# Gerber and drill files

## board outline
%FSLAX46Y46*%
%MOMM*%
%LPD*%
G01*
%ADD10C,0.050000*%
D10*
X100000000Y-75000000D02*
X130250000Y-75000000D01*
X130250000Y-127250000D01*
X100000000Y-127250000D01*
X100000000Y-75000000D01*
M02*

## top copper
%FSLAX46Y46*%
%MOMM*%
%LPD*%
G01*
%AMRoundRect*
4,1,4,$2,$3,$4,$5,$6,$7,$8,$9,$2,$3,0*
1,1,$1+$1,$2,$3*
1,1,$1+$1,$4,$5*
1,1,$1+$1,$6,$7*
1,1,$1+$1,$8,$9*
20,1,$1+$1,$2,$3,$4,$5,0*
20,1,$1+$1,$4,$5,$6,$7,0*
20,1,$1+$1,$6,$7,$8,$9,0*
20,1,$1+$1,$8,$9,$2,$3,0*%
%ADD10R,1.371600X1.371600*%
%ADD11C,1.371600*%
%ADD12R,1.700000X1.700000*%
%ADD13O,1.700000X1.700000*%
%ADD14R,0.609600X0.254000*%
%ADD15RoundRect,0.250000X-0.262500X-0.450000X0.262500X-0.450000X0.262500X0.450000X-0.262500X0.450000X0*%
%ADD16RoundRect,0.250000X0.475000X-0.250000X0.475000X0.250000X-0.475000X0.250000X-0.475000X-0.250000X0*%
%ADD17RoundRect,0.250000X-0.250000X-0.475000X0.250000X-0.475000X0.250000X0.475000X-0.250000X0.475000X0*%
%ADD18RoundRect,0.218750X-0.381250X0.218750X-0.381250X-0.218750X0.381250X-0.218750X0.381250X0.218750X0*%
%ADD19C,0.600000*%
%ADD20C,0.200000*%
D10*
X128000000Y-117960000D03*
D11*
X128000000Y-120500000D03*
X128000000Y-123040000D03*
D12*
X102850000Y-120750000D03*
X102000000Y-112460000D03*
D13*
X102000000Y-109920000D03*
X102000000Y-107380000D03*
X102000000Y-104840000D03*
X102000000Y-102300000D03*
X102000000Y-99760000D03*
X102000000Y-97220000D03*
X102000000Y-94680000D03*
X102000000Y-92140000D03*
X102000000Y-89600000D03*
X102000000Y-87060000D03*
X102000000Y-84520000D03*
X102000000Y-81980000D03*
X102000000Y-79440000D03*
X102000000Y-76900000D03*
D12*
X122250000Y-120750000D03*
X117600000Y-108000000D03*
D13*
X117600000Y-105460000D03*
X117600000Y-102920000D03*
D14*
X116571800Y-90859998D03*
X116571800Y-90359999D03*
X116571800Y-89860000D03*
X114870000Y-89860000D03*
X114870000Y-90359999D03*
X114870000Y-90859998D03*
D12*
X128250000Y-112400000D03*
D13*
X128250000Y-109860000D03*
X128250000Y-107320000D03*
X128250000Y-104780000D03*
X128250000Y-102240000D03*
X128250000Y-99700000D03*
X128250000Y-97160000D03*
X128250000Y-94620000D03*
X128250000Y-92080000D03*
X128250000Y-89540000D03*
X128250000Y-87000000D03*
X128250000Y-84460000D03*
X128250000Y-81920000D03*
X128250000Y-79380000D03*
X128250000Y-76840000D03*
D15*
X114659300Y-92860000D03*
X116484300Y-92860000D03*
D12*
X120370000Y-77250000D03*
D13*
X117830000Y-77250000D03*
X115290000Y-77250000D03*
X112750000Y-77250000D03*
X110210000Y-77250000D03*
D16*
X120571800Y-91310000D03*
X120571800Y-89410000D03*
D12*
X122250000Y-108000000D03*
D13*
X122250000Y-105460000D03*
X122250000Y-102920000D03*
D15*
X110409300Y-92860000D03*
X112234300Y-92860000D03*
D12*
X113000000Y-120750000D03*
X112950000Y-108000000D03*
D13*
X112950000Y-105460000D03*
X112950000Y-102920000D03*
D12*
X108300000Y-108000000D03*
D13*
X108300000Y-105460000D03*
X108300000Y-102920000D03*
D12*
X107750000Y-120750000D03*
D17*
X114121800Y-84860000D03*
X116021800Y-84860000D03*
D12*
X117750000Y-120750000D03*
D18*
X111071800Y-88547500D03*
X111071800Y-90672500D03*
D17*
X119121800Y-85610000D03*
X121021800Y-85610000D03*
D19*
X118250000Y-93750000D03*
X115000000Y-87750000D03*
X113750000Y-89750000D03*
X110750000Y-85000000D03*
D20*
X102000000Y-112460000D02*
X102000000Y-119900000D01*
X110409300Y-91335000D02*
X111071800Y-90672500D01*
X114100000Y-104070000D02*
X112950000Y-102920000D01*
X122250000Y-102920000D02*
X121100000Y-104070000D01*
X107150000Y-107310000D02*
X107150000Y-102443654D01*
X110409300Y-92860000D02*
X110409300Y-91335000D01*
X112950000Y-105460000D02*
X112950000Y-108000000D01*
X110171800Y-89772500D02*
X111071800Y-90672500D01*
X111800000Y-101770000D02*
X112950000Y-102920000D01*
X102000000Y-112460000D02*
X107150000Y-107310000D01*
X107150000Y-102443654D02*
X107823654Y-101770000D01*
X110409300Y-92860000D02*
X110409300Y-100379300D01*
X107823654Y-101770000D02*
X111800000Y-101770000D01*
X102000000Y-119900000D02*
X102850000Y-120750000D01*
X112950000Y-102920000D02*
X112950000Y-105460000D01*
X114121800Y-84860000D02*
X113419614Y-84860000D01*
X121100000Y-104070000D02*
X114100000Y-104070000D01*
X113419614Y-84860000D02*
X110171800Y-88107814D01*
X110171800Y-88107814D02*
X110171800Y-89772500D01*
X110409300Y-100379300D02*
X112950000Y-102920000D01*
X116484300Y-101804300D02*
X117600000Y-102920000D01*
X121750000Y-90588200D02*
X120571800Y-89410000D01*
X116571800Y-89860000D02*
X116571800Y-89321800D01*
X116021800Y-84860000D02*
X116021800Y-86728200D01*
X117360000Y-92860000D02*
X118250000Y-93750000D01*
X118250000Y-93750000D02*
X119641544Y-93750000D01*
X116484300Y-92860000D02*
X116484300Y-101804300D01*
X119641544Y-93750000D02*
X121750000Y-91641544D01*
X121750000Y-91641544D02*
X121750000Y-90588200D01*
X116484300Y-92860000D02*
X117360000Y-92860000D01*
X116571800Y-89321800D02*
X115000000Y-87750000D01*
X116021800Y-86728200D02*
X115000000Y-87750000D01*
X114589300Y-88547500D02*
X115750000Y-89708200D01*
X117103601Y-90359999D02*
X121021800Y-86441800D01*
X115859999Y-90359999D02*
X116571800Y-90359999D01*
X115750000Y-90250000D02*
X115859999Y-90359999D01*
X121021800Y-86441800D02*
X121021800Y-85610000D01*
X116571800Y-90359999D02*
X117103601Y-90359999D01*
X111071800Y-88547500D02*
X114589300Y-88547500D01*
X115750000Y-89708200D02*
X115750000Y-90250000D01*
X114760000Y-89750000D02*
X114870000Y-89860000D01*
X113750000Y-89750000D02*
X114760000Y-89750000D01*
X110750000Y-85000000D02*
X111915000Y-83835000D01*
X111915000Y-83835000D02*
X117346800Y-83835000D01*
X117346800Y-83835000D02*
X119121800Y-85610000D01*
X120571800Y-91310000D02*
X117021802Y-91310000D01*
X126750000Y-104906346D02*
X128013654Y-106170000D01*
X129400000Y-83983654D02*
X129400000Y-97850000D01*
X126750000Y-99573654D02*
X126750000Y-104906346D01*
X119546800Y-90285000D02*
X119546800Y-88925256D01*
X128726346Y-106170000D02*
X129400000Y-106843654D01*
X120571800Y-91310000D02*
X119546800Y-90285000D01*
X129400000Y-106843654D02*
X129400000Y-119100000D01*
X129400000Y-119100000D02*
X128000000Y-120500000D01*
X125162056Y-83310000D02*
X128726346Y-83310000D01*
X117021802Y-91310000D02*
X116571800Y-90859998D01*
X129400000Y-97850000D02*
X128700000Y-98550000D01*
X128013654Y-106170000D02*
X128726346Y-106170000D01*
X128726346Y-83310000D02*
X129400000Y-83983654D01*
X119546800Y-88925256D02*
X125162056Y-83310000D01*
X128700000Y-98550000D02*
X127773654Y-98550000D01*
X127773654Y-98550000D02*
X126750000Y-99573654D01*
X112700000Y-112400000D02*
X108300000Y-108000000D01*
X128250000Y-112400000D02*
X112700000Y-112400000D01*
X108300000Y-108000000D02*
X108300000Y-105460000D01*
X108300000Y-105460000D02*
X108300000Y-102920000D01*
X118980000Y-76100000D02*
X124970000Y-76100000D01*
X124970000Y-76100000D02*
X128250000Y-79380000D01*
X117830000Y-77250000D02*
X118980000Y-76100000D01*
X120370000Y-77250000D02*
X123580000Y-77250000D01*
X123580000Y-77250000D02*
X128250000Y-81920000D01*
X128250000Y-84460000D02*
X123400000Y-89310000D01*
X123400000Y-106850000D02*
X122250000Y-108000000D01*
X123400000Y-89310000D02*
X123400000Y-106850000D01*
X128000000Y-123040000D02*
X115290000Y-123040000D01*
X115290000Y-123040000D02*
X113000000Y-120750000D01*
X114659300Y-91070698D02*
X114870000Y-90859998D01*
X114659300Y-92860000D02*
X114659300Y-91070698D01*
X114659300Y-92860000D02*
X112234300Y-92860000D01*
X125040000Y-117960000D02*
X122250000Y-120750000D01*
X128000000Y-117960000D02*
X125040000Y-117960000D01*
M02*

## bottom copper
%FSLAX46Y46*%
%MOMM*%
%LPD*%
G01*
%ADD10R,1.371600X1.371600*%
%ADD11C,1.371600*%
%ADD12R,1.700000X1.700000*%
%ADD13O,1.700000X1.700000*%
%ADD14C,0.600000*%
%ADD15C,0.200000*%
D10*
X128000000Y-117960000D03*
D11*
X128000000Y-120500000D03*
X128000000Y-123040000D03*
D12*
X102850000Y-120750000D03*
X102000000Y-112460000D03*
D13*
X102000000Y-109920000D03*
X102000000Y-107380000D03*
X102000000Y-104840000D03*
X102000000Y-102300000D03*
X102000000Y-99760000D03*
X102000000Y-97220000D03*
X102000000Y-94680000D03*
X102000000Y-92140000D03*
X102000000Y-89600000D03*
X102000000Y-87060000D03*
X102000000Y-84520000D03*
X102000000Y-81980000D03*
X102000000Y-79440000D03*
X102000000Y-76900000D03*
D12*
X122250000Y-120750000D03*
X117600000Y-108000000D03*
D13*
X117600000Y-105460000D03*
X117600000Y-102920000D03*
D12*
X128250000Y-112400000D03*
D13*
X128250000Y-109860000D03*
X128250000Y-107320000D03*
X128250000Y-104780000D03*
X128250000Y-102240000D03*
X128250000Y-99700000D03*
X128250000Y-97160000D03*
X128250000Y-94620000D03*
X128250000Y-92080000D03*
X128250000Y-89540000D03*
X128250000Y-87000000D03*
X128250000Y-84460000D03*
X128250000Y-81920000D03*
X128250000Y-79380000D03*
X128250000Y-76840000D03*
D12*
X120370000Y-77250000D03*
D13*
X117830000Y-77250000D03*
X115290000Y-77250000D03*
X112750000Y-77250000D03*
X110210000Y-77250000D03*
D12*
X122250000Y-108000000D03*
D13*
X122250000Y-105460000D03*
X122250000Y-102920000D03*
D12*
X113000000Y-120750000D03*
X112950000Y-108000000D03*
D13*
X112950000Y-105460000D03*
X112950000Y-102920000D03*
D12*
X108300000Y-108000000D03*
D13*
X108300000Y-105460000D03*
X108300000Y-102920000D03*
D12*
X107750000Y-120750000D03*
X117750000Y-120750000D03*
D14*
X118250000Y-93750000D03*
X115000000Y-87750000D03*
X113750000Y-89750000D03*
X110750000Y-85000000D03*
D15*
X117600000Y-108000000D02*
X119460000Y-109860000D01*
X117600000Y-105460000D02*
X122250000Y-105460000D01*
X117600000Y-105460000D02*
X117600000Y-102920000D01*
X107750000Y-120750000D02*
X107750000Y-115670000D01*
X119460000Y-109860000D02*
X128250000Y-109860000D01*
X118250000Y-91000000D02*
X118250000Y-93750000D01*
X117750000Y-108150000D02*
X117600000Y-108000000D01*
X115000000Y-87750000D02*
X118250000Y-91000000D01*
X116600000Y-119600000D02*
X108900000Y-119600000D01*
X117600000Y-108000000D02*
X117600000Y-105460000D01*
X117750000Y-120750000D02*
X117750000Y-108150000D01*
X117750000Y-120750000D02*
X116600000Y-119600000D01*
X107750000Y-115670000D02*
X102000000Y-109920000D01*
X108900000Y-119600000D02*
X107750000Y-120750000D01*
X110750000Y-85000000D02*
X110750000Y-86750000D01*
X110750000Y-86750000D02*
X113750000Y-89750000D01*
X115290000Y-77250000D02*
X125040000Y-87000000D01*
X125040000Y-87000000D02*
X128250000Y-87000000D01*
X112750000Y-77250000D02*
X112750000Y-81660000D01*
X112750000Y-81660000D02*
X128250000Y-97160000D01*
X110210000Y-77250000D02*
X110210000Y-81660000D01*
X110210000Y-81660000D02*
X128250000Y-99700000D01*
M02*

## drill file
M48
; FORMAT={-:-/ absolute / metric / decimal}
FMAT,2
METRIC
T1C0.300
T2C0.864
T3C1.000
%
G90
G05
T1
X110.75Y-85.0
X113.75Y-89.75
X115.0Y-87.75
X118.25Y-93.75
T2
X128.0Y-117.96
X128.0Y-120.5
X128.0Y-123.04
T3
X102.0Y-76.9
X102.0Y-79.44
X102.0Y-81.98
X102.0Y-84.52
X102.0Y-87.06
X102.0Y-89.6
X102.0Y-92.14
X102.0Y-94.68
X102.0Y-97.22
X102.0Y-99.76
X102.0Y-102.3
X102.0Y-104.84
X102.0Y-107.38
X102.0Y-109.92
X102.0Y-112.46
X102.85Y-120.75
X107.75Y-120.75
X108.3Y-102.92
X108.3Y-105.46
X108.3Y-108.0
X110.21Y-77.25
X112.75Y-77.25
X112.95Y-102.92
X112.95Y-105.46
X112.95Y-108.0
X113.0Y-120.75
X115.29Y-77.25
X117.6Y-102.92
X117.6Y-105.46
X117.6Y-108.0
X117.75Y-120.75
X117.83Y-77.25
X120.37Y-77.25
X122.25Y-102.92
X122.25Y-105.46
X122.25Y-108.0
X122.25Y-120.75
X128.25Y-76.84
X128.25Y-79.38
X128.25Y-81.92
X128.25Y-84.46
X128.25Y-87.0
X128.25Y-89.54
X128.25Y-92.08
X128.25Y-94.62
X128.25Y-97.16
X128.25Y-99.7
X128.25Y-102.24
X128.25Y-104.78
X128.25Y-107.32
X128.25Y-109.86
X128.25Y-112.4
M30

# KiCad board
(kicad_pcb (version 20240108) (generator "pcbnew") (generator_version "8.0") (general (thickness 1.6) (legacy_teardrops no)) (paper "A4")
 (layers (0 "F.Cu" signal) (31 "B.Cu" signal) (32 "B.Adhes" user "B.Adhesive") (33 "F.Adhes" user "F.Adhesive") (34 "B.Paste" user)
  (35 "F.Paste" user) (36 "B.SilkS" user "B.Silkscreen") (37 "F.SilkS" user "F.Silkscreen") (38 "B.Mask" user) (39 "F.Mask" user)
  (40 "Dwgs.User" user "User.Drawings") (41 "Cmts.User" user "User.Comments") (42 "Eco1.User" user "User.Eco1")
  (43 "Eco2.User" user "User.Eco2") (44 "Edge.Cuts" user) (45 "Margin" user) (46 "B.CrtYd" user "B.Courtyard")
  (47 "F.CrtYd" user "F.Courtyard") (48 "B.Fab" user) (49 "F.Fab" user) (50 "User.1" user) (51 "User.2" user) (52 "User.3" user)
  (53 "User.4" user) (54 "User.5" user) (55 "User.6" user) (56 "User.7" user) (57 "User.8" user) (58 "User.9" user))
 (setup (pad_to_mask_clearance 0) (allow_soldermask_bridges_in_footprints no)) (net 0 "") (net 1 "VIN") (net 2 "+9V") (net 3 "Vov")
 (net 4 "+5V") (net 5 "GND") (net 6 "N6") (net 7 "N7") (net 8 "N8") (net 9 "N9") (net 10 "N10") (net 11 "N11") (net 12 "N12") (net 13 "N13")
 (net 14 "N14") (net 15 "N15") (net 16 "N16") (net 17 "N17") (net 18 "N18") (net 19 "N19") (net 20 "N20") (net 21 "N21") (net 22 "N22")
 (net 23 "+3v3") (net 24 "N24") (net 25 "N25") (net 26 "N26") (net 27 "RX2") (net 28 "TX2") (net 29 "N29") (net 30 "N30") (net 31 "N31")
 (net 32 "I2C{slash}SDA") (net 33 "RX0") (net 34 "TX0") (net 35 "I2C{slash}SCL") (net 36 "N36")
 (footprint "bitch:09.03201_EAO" (layer "F.Cu") (at 128 117.96)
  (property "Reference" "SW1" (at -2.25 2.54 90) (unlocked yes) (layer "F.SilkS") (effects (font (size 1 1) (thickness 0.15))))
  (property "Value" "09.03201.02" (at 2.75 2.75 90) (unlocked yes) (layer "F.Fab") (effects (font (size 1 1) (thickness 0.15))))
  (pad "1" thru_hole rect (at 0 0) (size 1.3716 1.3716) (drill 0.8636) (layers "*.Cu" "*.Mask") (remove_unused_layers no) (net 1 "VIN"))
  (pad "2" thru_hole circle (at 0 2.54) (size 1.3716 1.3716) (drill 0.8636) (layers "*.Cu" "*.Mask") (remove_unused_layers no) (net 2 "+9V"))
  (pad "3" thru_hole circle (at 0 5.08) (size 1.3716 1.3716) (drill 0.8636) (layers "*.Cu" "*.Mask") (remove_unused_layers no) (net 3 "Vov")))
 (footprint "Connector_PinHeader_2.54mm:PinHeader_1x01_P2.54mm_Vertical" (layer "F.Cu") (at 102.85 120.75 90)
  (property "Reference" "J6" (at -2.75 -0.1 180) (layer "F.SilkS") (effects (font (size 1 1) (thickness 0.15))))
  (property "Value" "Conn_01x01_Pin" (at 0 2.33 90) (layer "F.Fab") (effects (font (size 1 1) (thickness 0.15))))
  (pad "1" thru_hole rect (at 0 0 90) (size 1.7 1.7) (drill 1) (layers "*.Cu" "*.Mask") (remove_unused_layers no) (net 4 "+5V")))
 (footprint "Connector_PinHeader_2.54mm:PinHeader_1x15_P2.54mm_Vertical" (layer "F.Cu") (at 102 112.46 180)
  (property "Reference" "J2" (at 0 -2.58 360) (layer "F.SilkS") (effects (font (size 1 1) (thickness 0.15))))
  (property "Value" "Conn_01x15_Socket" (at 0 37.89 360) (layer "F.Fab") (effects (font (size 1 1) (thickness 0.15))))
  (pad "1" thru_hole rect (at 0 0 180) (size 1.7 1.7) (drill 1) (layers "*.Cu" "*.Mask") (remove_unused_layers no) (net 4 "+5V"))
  (pad "2" thru_hole oval (at 0 2.54 180) (size 1.7 1.7) (drill 1) (layers "*.Cu" "*.Mask") (remove_unused_layers no) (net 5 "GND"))
  (pad "3" thru_hole oval (at 0 5.08 180) (size 1.7 1.7) (drill 1) (layers "*.Cu" "*.Mask") (remove_unused_layers no) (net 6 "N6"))
  (pad "4" thru_hole oval (at 0 7.62 180) (size 1.7 1.7) (drill 1) (layers "*.Cu" "*.Mask") (remove_unused_layers no) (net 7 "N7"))
  (pad "5" thru_hole oval (at 0 10.16 180) (size 1.7 1.7) (drill 1) (layers "*.Cu" "*.Mask") (remove_unused_layers no) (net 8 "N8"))
  (pad "6" thru_hole oval (at 0 12.7 180) (size 1.7 1.7) (drill 1) (layers "*.Cu" "*.Mask") (remove_unused_layers no) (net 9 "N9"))
  (pad "7" thru_hole oval (at 0 15.24 180) (size 1.7 1.7) (drill 1) (layers "*.Cu" "*.Mask") (remove_unused_layers no) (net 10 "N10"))
  (pad "8" thru_hole oval (at 0 17.78 180) (size 1.7 1.7) (drill 1) (layers "*.Cu" "*.Mask") (remove_unused_layers no) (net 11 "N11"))
  (pad "9" thru_hole oval (at 0 20.32 180) (size 1.7 1.7) (drill 1) (layers "*.Cu" "*.Mask") (remove_unused_layers no) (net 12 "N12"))
  (pad "10" thru_hole oval (at 0 22.86 180) (size 1.7 1.7) (drill 1) (layers "*.Cu" "*.Mask") (remove_unused_layers no) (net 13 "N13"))
  (pad "11" thru_hole oval (at 0 25.4 180) (size 1.7 1.7) (drill 1) (layers "*.Cu" "*.Mask") (remove_unused_layers no) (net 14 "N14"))
  (pad "12" thru_hole oval (at 0 27.94 180) (size 1.7 1.7) (drill 1) (layers "*.Cu" "*.Mask") (remove_unused_layers no) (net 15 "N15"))
  (pad "13" thru_hole oval (at 0 30.48 180) (size 1.7 1.7) (drill 1) (layers "*.Cu" "*.Mask") (remove_unused_layers no) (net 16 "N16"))
  (pad "14" thru_hole oval (at 0 33.02 180) (size 1.7 1.7) (drill 1) (layers "*.Cu" "*.Mask") (remove_unused_layers no) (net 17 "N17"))
  (pad "15" thru_hole oval (at 0 35.56 180) (size 1.7 1.7) (drill 1) (layers "*.Cu" "*.Mask") (remove_unused_layers no) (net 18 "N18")))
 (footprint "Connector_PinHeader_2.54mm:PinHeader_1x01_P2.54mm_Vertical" (layer "F.Cu") (at 122.25 120.75 90)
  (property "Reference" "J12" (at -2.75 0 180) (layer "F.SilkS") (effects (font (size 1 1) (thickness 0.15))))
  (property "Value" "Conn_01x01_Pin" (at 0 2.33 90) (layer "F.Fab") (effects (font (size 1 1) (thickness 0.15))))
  (pad "1" thru_hole rect (at 0 0 90) (size 1.7 1.7) (drill 1) (layers "*.Cu" "*.Mask") (remove_unused_layers no) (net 1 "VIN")))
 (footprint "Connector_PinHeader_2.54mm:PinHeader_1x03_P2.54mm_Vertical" (layer "F.Cu") (at 117.6 108 180)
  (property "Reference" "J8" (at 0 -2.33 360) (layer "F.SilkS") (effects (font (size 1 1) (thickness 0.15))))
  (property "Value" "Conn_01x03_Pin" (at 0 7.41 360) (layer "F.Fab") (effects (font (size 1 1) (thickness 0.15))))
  (pad "1" thru_hole rect (at 0 0 180) (size 1.7 1.7) (drill 1) (layers "*.Cu" "*.Mask") (remove_unused_layers no) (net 5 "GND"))
  (pad "2" thru_hole oval (at 0 2.54 180) (size 1.7 1.7) (drill 1) (layers "*.Cu" "*.Mask") (remove_unused_layers no) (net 5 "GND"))
  (pad "3" thru_hole oval (at 0 5.08 180) (size 1.7 1.7) (drill 1) (layers "*.Cu" "*.Mask") (remove_unused_layers no) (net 5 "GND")))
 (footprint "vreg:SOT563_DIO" (layer "F.Cu") (at 115.7209 90.359999 180)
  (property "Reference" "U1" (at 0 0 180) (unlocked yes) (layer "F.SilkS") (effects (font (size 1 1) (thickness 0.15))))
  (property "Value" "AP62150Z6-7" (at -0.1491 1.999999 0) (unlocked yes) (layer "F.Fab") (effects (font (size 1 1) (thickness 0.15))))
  (pad "1" smd rect (at -0.8509 -0.499999 180) (size 0.6096 0.254) (layers "F.Cu" "F.Paste" "F.Mask") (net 2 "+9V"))
  (pad "2" smd rect (at -0.8509 0 180) (size 0.6096 0.254) (layers "F.Cu" "F.Paste" "F.Mask") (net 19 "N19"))
  (pad "3" smd rect (at -0.8509 0.499999 180) (size 0.6096 0.254) (layers "F.Cu" "F.Paste" "F.Mask") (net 5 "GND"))
  (pad "4" smd rect (at 0.8509 0.499999 180) (size 0.6096 0.254) (layers "F.Cu" "F.Paste" "F.Mask") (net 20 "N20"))
  (pad "5" smd rect (at 0.8509 0 180) (size 0.6096 0.254) (layers "F.Cu" "F.Paste" "F.Mask") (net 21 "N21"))
  (pad "6" smd rect (at 0.8509 -0.499999 180) (size 0.6096 0.254) (layers "F.Cu" "F.Paste" "F.Mask") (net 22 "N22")))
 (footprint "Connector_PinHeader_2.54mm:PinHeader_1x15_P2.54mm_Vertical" (layer "F.Cu") (at 128.25 112.4 180)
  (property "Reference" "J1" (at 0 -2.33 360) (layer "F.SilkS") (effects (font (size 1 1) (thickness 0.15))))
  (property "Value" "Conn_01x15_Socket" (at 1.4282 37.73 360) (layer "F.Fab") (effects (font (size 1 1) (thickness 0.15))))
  (pad "1" thru_hole rect (at 0 0 180) (size 1.7 1.7) (drill 1) (layers "*.Cu" "*.Mask") (remove_unused_layers no) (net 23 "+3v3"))
  (pad "2" thru_hole oval (at 0 2.54 180) (size 1.7 1.7) (drill 1) (layers "*.Cu" "*.Mask") (remove_unused_layers no) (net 5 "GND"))
  (pad "3" thru_hole oval (at 0 5.08 180) (size 1.7 1.7) (drill 1) (layers "*.Cu" "*.Mask") (remove_unused_layers no) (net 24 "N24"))
  (pad "4" thru_hole oval (at 0 7.62 180) (size 1.7 1.7) (drill 1) (layers "*.Cu" "*.Mask") (remove_unused_layers no) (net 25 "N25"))
  (pad "5" thru_hole oval (at 0 10.16 180) (size 1.7 1.7) (drill 1) (layers "*.Cu" "*.Mask") (remove_unused_layers no) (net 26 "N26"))
  (pad "6" thru_hole oval (at 0 12.7 180) (size 1.7 1.7) (drill 1) (layers "*.Cu" "*.Mask") (remove_unused_layers no) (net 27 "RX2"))
  (pad "7" thru_hole oval (at 0 15.24 180) (size 1.7 1.7) (drill 1) (layers "*.Cu" "*.Mask") (remove_unused_layers no) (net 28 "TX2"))
  (pad "8" thru_hole oval (at 0 17.78 180) (size 1.7 1.7) (drill 1) (layers "*.Cu" "*.Mask") (remove_unused_layers no) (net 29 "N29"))
  (pad "9" thru_hole oval (at 0 20.32 180) (size 1.7 1.7) (drill 1) (layers "*.Cu" "*.Mask") (remove_unused_layers no) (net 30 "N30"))
  (pad "10" thru_hole oval (at 0 22.86 180) (size 1.7 1.7) (drill 1) (layers "*.Cu" "*.Mask") (remove_unused_layers no) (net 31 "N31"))
  (pad "11" thru_hole oval (at 0 25.4 180) (size 1.7 1.7) (drill 1) (layers "*.Cu" "*.Mask") (remove_unused_layers no)
   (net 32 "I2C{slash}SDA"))
  (pad "12" thru_hole oval (at 0 27.94 180) (size 1.7 1.7) (drill 1) (layers "*.Cu" "*.Mask") (remove_unused_layers no) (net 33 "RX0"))
  (pad "13" thru_hole oval (at 0 30.48 180) (size 1.7 1.7) (drill 1) (layers "*.Cu" "*.Mask") (remove_unused_layers no) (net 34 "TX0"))
  (pad "14" thru_hole oval (at 0 33.02 180) (size 1.7 1.7) (drill 1) (layers "*.Cu" "*.Mask") (remove_unused_layers no)
   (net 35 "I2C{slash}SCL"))
  (pad "15" thru_hole oval (at 0 35.56 180) (size 1.7 1.7) (drill 1) (layers "*.Cu" "*.Mask") (remove_unused_layers no) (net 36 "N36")))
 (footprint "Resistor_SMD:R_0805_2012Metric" (layer "F.Cu") (at 115.5718 92.86)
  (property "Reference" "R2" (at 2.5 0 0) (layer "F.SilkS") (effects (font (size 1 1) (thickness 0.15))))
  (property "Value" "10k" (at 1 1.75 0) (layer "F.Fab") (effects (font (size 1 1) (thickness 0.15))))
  (pad "1" smd roundrect (at -0.9125 0) (size 1.025 1.4) (layers "F.Cu" "F.Paste" "F.Mask") (roundrect_rratio 0.243902) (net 22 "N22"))
  (pad "2" smd roundrect (at 0.9125 0) (size 1.025 1.4) (layers "F.Cu" "F.Paste" "F.Mask") (roundrect_rratio 0.243902) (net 5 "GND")))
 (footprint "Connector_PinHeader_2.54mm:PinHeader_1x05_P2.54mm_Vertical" (layer "F.Cu") (at 120.37 77.25 -90)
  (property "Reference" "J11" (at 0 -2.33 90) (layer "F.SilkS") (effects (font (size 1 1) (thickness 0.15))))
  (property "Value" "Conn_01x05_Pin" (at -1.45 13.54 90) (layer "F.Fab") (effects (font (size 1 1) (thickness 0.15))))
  (pad "1" thru_hole rect (at 0 0 270) (size 1.7 1.7) (drill 1) (layers "*.Cu" "*.Mask") (remove_unused_layers no) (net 34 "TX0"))
  (pad "2" thru_hole oval (at 0 2.54 270) (size 1.7 1.7) (drill 1) (layers "*.Cu" "*.Mask") (remove_unused_layers no)
   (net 35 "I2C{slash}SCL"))
  (pad "3" thru_hole oval (at 0 5.08 270) (size 1.7 1.7) (drill 1) (layers "*.Cu" "*.Mask") (remove_unused_layers no)
   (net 32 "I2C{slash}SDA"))
  (pad "4" thru_hole oval (at 0 7.62 270) (size 1.7 1.7) (drill 1) (layers "*.Cu" "*.Mask") (remove_unused_layers no) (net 28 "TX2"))
  (pad "5" thru_hole oval (at 0 10.16 270) (size 1.7 1.7) (drill 1) (layers "*.Cu" "*.Mask") (remove_unused_layers no) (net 27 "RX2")))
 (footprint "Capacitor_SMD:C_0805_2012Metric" (layer "F.Cu") (at 120.5718 90.36 90)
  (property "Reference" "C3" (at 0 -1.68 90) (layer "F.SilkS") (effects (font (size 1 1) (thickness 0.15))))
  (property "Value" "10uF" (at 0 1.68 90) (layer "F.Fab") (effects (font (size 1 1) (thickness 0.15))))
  (pad "1" smd roundrect (at -0.95 0 90) (size 1 1.45) (layers "F.Cu" "F.Paste" "F.Mask") (roundrect_rratio 0.25) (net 2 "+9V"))
  (pad "2" smd roundrect (at 0.95 0 90) (size 1 1.45) (layers "F.Cu" "F.Paste" "F.Mask") (roundrect_rratio 0.25) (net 5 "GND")))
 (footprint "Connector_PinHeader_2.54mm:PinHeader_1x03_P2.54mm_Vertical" (layer "F.Cu") (at 122.25 108 180)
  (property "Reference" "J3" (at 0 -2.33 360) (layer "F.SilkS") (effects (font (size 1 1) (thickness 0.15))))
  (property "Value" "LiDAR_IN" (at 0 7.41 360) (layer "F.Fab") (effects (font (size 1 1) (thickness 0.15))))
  (pad "1" thru_hole rect (at 0 0 180) (size 1.7 1.7) (drill 1) (layers "*.Cu" "*.Mask") (remove_unused_layers no) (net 33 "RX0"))
  (pad "2" thru_hole oval (at 0 2.54 180) (size 1.7 1.7) (drill 1) (layers "*.Cu" "*.Mask") (remove_unused_layers no) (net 5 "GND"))
  (pad "3" thru_hole oval (at 0 5.08 180) (size 1.7 1.7) (drill 1) (layers "*.Cu" "*.Mask") (remove_unused_layers no) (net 4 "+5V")))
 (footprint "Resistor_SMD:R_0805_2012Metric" (layer "F.Cu") (at 111.3218 92.86)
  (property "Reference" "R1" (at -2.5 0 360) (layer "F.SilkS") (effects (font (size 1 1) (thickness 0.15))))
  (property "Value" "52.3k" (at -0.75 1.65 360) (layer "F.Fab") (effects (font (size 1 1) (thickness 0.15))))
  (pad "1" smd roundrect (at -0.9125 0) (size 1.025 1.4) (layers "F.Cu" "F.Paste" "F.Mask") (roundrect_rratio 0.243902) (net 4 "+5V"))
  (pad "2" smd roundrect (at 0.9125 0) (size 1.025 1.4) (layers "F.Cu" "F.Paste" "F.Mask") (roundrect_rratio 0.243902) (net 22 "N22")))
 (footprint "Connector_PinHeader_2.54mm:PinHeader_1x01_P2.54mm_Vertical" (layer "F.Cu") (at 113 120.75 90)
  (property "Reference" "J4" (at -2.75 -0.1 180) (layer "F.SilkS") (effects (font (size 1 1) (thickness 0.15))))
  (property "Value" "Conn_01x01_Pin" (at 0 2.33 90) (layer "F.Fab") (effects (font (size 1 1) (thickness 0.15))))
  (pad "1" thru_hole rect (at 0 0 90) (size 1.7 1.7) (drill 1) (layers "*.Cu" "*.Mask") (remove_unused_layers no) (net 3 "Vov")))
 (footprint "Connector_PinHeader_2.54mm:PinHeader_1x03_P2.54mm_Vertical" (layer "F.Cu") (at 112.95 108 180)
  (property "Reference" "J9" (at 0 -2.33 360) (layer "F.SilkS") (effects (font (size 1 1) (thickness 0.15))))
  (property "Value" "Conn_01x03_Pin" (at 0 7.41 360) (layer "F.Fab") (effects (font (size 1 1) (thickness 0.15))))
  (pad "1" thru_hole rect (at 0 0 180) (size 1.7 1.7) (drill 1) (layers "*.Cu" "*.Mask") (remove_unused_layers no) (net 4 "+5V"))
  (pad "2" thru_hole oval (at 0 2.54 180) (size 1.7 1.7) (drill 1) (layers "*.Cu" "*.Mask") (remove_unused_layers no) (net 4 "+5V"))
  (pad "3" thru_hole oval (at 0 5.08 180) (size 1.7 1.7) (drill 1) (layers "*.Cu" "*.Mask") (remove_unused_layers no) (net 4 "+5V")))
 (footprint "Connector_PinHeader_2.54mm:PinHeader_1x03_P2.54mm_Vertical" (layer "F.Cu") (at 108.3 108 180)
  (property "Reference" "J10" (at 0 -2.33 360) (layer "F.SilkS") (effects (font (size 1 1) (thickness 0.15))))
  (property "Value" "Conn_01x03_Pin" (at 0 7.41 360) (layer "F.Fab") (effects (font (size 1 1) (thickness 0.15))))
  (pad "1" thru_hole rect (at 0 0 180) (size 1.7 1.7) (drill 1) (layers "*.Cu" "*.Mask") (remove_unused_layers no) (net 23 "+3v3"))
  (pad "2" thru_hole oval (at 0 2.54 180) (size 1.7 1.7) (drill 1) (layers "*.Cu" "*.Mask") (remove_unused_layers no) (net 23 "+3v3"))
  (pad "3" thru_hole oval (at 0 5.08 180) (size 1.7 1.7) (drill 1) (layers "*.Cu" "*.Mask") (remove_unused_layers no) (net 23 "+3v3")))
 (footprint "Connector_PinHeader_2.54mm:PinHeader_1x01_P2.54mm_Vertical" (layer "F.Cu") (at 107.75 120.75 90)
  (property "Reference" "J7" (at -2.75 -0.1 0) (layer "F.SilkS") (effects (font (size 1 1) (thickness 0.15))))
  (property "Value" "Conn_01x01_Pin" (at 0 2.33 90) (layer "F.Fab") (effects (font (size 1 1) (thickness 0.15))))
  (pad "1" thru_hole rect (at 0 0 90) (size 1.7 1.7) (drill 1) (layers "*.Cu" "*.Mask") (remove_unused_layers no) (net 5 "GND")))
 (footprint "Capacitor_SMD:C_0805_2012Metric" (layer "F.Cu") (at 115.0718 84.86)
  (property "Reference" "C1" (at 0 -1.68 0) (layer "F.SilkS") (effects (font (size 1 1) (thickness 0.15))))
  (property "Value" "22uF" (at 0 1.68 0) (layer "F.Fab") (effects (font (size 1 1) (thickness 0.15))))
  (pad "1" smd roundrect (at -0.95 0) (size 1 1.45) (layers "F.Cu" "F.Paste" "F.Mask") (roundrect_rratio 0.25) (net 4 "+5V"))
  (pad "2" smd roundrect (at 0.95 0) (size 1 1.45) (layers "F.Cu" "F.Paste" "F.Mask") (roundrect_rratio 0.25) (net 5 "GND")))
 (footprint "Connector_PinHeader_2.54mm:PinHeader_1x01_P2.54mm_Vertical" (layer "F.Cu") (at 117.75 120.75 90)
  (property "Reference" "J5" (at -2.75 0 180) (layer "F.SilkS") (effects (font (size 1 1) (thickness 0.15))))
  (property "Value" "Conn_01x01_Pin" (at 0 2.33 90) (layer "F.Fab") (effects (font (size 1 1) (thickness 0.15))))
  (pad "1" thru_hole rect (at 0 0 90) (size 1.7 1.7) (drill 1) (layers "*.Cu" "*.Mask") (remove_unused_layers no) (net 5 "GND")))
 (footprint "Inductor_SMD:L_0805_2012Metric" (layer "F.Cu") (at 111.0718 89.61 -90)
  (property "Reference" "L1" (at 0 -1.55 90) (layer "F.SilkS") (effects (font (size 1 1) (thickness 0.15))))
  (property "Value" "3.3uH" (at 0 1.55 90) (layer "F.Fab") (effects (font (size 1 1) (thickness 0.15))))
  (pad "1" smd roundrect (at -1.0625 0 270) (size 0.875 1.2) (layers "F.Cu" "F.Paste" "F.Mask") (roundrect_rratio 0.25) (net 19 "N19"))
  (pad "2" smd roundrect (at 1.0625 0 270) (size 0.875 1.2) (layers "F.Cu" "F.Paste" "F.Mask") (roundrect_rratio 0.25) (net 4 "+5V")))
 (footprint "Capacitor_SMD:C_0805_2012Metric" (layer "F.Cu") (at 120.0718 85.61)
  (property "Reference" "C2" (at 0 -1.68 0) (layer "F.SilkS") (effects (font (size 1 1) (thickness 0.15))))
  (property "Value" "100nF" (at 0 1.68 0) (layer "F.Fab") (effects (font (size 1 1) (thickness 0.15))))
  (pad "1" smd roundrect (at -0.95 0) (size 1 1.45) (layers "F.Cu" "F.Paste" "F.Mask") (roundrect_rratio 0.25) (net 20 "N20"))
  (pad "2" smd roundrect (at 0.95 0) (size 1 1.45) (layers "F.Cu" "F.Paste" "F.Mask") (roundrect_rratio 0.25) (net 19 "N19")))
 (gr_rect (start 100 75) (end 130.25 127.25) (stroke (width 0.05) (type default)) (fill none) (layer "Edge.Cuts"))
 (segment (start 102 112.46) (end 102 119.9) (width 0.2) (layer "F.Cu") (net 4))
 (segment (start 110.4093 91.335) (end 111.0718 90.6725) (width 0.2) (layer "F.Cu") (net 4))
 (segment (start 114.1 104.07) (end 112.95 102.92) (width 0.2) (layer "F.Cu") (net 4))
 (segment (start 122.25 102.92) (end 121.1 104.07) (width 0.2) (layer "F.Cu") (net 4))
 (segment (start 107.15 107.31) (end 107.15 102.443654) (width 0.2) (layer "F.Cu") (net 4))
 (segment (start 110.4093 92.86) (end 110.4093 91.335) (width 0.2) (layer "F.Cu") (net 4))
 (segment (start 112.95 105.46) (end 112.95 108) (width 0.2) (layer "F.Cu") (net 4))
 (segment (start 110.1718 89.7725) (end 111.0718 90.6725) (width 0.2) (layer "F.Cu") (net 4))
 (segment (start 111.8 101.77) (end 112.95 102.92) (width 0.2) (layer "F.Cu") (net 4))
 (segment (start 102 112.46) (end 107.15 107.31) (width 0.2) (layer "F.Cu") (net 4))
 (segment (start 107.15 102.443654) (end 107.823654 101.77) (width 0.2) (layer "F.Cu") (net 4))
 (segment (start 110.4093 92.86) (end 110.4093 100.3793) (width 0.2) (layer "F.Cu") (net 4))
 (segment (start 107.823654 101.77) (end 111.8 101.77) (width 0.2) (layer "F.Cu") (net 4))
 (segment (start 102 119.9) (end 102.85 120.75) (width 0.2) (layer "F.Cu") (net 4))
 (segment (start 112.95 102.92) (end 112.95 105.46) (width 0.2) (layer "F.Cu") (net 4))
 (segment (start 114.1218 84.86) (end 113.419614 84.86) (width 0.2) (layer "F.Cu") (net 4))
 (segment (start 121.1 104.07) (end 114.1 104.07) (width 0.2) (layer "F.Cu") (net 4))
 (segment (start 113.419614 84.86) (end 110.1718 88.107814) (width 0.2) (layer "F.Cu") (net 4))
 (segment (start 110.1718 88.107814) (end 110.1718 89.7725) (width 0.2) (layer "F.Cu") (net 4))
 (segment (start 110.4093 100.3793) (end 112.95 102.92) (width 0.2) (layer "F.Cu") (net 4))
 (segment (start 116.4843 101.8043) (end 117.6 102.92) (width 0.2) (layer "F.Cu") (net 5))
 (segment (start 121.75 90.5882) (end 120.5718 89.41) (width 0.2) (layer "F.Cu") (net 5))
 (segment (start 116.5718 89.86) (end 116.5718 89.3218) (width 0.2) (layer "F.Cu") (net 5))
 (segment (start 116.0218 84.86) (end 116.0218 86.7282) (width 0.2) (layer "F.Cu") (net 5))
 (segment (start 117.36 92.86) (end 118.25 93.75) (width 0.2) (layer "F.Cu") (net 5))
 (segment (start 118.25 93.75) (end 119.641544 93.75) (width 0.2) (layer "F.Cu") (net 5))
 (segment (start 116.4843 92.86) (end 116.4843 101.8043) (width 0.2) (layer "F.Cu") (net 5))
 (segment (start 119.641544 93.75) (end 121.75 91.641544) (width 0.2) (layer "F.Cu") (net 5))
 (segment (start 121.75 91.641544) (end 121.75 90.5882) (width 0.2) (layer "F.Cu") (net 5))
 (segment (start 116.4843 92.86) (end 117.36 92.86) (width 0.2) (layer "F.Cu") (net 5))
 (segment (start 116.5718 89.3218) (end 115 87.75) (width 0.2) (layer "F.Cu") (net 5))
 (segment (start 116.0218 86.7282) (end 115 87.75) (width 0.2) (layer "F.Cu") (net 5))
 (via (at 118.25 93.75) (size 0.6) (drill 0.3) (layers "F.Cu" "B.Cu") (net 5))
 (via (at 115 87.75) (size 0.6) (drill 0.3) (layers "F.Cu" "B.Cu") (free yes) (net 5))
 (segment (start 117.6 108) (end 119.46 109.86) (width 0.2) (layer "B.Cu") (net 5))
 (segment (start 117.6 105.46) (end 122.25 105.46) (width 0.2) (layer "B.Cu") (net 5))
 (segment (start 117.6 105.46) (end 117.6 102.92) (width 0.2) (layer "B.Cu") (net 5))
 (segment (start 107.75 120.75) (end 107.75 115.67) (width 0.2) (layer "B.Cu") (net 5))
 (segment (start 119.46 109.86) (end 128.25 109.86) (width 0.2) (layer "B.Cu") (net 5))
 (segment (start 118.25 91) (end 118.25 93.75) (width 0.2) (layer "B.Cu") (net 5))
 (segment (start 117.75 108.15) (end 117.6 108) (width 0.2) (layer "B.Cu") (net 5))
 (segment (start 115 87.75) (end 118.25 91) (width 0.2) (layer "B.Cu") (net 5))
 (segment (start 116.6 119.6) (end 108.9 119.6) (width 0.2) (layer "B.Cu") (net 5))
 (segment (start 117.6 108) (end 117.6 105.46) (width 0.2) (layer "B.Cu") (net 5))
 (segment (start 117.75 120.75) (end 117.75 108.15) (width 0.2) (layer "B.Cu") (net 5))
 (segment (start 117.75 120.75) (end 116.6 119.6) (width 0.2) (layer "B.Cu") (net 5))
 (segment (start 107.75 115.67) (end 102 109.92) (width 0.2) (layer "B.Cu") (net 5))
 (segment (start 108.9 119.6) (end 107.75 120.75) (width 0.2) (layer "B.Cu") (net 5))
 (segment (start 114.5893 88.5475) (end 115.75 89.7082) (width 0.2) (layer "F.Cu") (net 19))
 (segment (start 117.103601 90.359999) (end 121.0218 86.4418) (width 0.2) (layer "F.Cu") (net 19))
 (segment (start 115.859999 90.359999) (end 116.5718 90.359999) (width 0.2) (layer "F.Cu") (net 19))
 (segment (start 115.75 90.25) (end 115.859999 90.359999) (width 0.2) (layer "F.Cu") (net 19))
 (segment (start 121.0218 86.4418) (end 121.0218 85.61) (width 0.2) (layer "F.Cu") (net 19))
 (segment (start 116.5718 90.359999) (end 117.103601 90.359999) (width 0.2) (layer "F.Cu") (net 19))
 (segment (start 111.0718 88.5475) (end 114.5893 88.5475) (width 0.2) (layer "F.Cu") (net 19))
 (segment (start 115.75 89.7082) (end 115.75 90.25) (width 0.2) (layer "F.Cu") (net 19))
 (segment (start 114.76 89.75) (end 114.87 89.86) (width 0.2) (layer "F.Cu") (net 20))
 (segment (start 113.75 89.75) (end 114.76 89.75) (width 0.2) (layer "F.Cu") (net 20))
 (segment (start 110.75 85) (end 111.915 83.835) (width 0.2) (layer "F.Cu") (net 20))
 (segment (start 111.915 83.835) (end 117.3468 83.835) (width 0.2) (layer "F.Cu") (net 20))
 (segment (start 117.3468 83.835) (end 119.1218 85.61) (width 0.2) (layer "F.Cu") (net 20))
 (via (at 113.75 89.75) (size 0.6) (drill 0.3) (layers "F.Cu" "B.Cu") (free yes) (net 20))
 (via (at 110.75 85) (size 0.6) (drill 0.3) (layers "F.Cu" "B.Cu") (free yes) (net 20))
 (segment (start 110.75 85) (end 110.75 86.75) (width 0.2) (layer "B.Cu") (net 20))
 (segment (start 110.75 86.75) (end 113.75 89.75) (width 0.2) (layer "B.Cu") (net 20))
 (segment (start 120.5718 91.31) (end 117.021802 91.31) (width 0.2) (layer "F.Cu") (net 2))
 (segment (start 126.75 104.906346) (end 128.013654 106.17) (width 0.2) (layer "F.Cu") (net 2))
 (segment (start 129.4 83.983654) (end 129.4 97.85) (width 0.2) (layer "F.Cu") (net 2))
 (segment (start 126.75 99.573654) (end 126.75 104.906346) (width 0.2) (layer "F.Cu") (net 2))
 (segment (start 119.5468 90.285) (end 119.5468 88.925256) (width 0.2) (layer "F.Cu") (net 2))
 (segment (start 128.726346 106.17) (end 129.4 106.843654) (width 0.2) (layer "F.Cu") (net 2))
 (segment (start 120.5718 91.31) (end 119.5468 90.285) (width 0.2) (layer "F.Cu") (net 2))
 (segment (start 129.4 106.843654) (end 129.4 119.1) (width 0.2) (layer "F.Cu") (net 2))
 (segment (start 129.4 119.1) (end 128 120.5) (width 0.2) (layer "F.Cu") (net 2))
 (segment (start 125.162056 83.31) (end 128.726346 83.31) (width 0.2) (layer "F.Cu") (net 2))
 (segment (start 117.021802 91.31) (end 116.5718 90.859998) (width 0.2) (layer "F.Cu") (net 2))
 (segment (start 129.4 97.85) (end 128.7 98.55) (width 0.2) (layer "F.Cu") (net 2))
 (segment (start 128.013654 106.17) (end 128.726346 106.17) (width 0.2) (layer "F.Cu") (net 2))
 (segment (start 128.726346 83.31) (end 129.4 83.983654) (width 0.2) (layer "F.Cu") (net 2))
 (segment (start 119.5468 88.925256) (end 125.162056 83.31) (width 0.2) (layer "F.Cu") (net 2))
 (segment (start 128.7 98.55) (end 127.773654 98.55) (width 0.2) (layer "F.Cu") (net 2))
 (segment (start 127.773654 98.55) (end 126.75 99.573654) (width 0.2) (layer "F.Cu") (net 2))
 (segment (start 115.29 77.25) (end 125.04 87) (width 0.2) (layer "B.Cu") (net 32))
 (segment (start 125.04 87) (end 128.25 87) (width 0.2) (layer "B.Cu") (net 32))
 (segment (start 112.7 112.4) (end 108.3 108) (width 0.2) (layer "F.Cu") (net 23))
 (segment (start 128.25 112.4) (end 112.7 112.4) (width 0.2) (layer "F.Cu") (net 23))
 (segment (start 108.3 108) (end 108.3 105.46) (width 0.2) (layer "F.Cu") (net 23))
 (segment (start 108.3 105.46) (end 108.3 102.92) (width 0.2) (layer "F.Cu") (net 23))
 (segment (start 112.75 77.25) (end 112.75 81.66) (width 0.2) (layer "B.Cu") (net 28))
 (segment (start 112.75 81.66) (end 128.25 97.16) (width 0.2) (layer "B.Cu") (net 28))
 (segment (start 110.21 77.25) (end 110.21 81.66) (width 0.2) (layer "B.Cu") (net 27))
 (segment (start 110.21 81.66) (end 128.25 99.7) (width 0.2) (layer "B.Cu") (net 27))
 (segment (start 118.98 76.1) (end 124.97 76.1) (width 0.2) (layer "F.Cu") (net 35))
 (segment (start 124.97 76.1) (end 128.25 79.38) (width 0.2) (layer "F.Cu") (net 35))
 (segment (start 117.83 77.25) (end 118.98 76.1) (width 0.2) (layer "F.Cu") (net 35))
 (segment (start 120.37 77.25) (end 123.58 77.25) (width 0.2) (layer "F.Cu") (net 34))
 (segment (start 123.58 77.25) (end 128.25 81.92) (width 0.2) (layer "F.Cu") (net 34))
 (segment (start 128.25 84.46) (end 123.4 89.31) (width 0.2) (layer "F.Cu") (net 33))
 (segment (start 123.4 106.85) (end 122.25 108) (width 0.2) (layer "F.Cu") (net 33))
 (segment (start 123.4 89.31) (end 123.4 106.85) (width 0.2) (layer "F.Cu") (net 33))
 (segment (start 128 123.04) (end 115.29 123.04) (width 0.2) (layer "F.Cu") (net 3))
 (segment (start 115.29 123.04) (end 113 120.75) (width 0.2) (layer "F.Cu") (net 3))
 (segment (start 114.6593 91.070698) (end 114.87 90.859998) (width 0.2) (layer "F.Cu") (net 22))
 (segment (start 114.6593 92.86) (end 114.6593 91.070698) (width 0.2) (layer "F.Cu") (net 22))
 (segment (start 114.6593 92.86) (end 112.2343 92.86) (width 0.2) (layer "F.Cu") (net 22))
 (segment (start 125.04 117.96) (end 122.25 120.75) (width 0.2) (layer "F.Cu") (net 1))
 (segment (start 128 117.96) (end 125.04 117.96) (width 0.2) (layer "F.Cu") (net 1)))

